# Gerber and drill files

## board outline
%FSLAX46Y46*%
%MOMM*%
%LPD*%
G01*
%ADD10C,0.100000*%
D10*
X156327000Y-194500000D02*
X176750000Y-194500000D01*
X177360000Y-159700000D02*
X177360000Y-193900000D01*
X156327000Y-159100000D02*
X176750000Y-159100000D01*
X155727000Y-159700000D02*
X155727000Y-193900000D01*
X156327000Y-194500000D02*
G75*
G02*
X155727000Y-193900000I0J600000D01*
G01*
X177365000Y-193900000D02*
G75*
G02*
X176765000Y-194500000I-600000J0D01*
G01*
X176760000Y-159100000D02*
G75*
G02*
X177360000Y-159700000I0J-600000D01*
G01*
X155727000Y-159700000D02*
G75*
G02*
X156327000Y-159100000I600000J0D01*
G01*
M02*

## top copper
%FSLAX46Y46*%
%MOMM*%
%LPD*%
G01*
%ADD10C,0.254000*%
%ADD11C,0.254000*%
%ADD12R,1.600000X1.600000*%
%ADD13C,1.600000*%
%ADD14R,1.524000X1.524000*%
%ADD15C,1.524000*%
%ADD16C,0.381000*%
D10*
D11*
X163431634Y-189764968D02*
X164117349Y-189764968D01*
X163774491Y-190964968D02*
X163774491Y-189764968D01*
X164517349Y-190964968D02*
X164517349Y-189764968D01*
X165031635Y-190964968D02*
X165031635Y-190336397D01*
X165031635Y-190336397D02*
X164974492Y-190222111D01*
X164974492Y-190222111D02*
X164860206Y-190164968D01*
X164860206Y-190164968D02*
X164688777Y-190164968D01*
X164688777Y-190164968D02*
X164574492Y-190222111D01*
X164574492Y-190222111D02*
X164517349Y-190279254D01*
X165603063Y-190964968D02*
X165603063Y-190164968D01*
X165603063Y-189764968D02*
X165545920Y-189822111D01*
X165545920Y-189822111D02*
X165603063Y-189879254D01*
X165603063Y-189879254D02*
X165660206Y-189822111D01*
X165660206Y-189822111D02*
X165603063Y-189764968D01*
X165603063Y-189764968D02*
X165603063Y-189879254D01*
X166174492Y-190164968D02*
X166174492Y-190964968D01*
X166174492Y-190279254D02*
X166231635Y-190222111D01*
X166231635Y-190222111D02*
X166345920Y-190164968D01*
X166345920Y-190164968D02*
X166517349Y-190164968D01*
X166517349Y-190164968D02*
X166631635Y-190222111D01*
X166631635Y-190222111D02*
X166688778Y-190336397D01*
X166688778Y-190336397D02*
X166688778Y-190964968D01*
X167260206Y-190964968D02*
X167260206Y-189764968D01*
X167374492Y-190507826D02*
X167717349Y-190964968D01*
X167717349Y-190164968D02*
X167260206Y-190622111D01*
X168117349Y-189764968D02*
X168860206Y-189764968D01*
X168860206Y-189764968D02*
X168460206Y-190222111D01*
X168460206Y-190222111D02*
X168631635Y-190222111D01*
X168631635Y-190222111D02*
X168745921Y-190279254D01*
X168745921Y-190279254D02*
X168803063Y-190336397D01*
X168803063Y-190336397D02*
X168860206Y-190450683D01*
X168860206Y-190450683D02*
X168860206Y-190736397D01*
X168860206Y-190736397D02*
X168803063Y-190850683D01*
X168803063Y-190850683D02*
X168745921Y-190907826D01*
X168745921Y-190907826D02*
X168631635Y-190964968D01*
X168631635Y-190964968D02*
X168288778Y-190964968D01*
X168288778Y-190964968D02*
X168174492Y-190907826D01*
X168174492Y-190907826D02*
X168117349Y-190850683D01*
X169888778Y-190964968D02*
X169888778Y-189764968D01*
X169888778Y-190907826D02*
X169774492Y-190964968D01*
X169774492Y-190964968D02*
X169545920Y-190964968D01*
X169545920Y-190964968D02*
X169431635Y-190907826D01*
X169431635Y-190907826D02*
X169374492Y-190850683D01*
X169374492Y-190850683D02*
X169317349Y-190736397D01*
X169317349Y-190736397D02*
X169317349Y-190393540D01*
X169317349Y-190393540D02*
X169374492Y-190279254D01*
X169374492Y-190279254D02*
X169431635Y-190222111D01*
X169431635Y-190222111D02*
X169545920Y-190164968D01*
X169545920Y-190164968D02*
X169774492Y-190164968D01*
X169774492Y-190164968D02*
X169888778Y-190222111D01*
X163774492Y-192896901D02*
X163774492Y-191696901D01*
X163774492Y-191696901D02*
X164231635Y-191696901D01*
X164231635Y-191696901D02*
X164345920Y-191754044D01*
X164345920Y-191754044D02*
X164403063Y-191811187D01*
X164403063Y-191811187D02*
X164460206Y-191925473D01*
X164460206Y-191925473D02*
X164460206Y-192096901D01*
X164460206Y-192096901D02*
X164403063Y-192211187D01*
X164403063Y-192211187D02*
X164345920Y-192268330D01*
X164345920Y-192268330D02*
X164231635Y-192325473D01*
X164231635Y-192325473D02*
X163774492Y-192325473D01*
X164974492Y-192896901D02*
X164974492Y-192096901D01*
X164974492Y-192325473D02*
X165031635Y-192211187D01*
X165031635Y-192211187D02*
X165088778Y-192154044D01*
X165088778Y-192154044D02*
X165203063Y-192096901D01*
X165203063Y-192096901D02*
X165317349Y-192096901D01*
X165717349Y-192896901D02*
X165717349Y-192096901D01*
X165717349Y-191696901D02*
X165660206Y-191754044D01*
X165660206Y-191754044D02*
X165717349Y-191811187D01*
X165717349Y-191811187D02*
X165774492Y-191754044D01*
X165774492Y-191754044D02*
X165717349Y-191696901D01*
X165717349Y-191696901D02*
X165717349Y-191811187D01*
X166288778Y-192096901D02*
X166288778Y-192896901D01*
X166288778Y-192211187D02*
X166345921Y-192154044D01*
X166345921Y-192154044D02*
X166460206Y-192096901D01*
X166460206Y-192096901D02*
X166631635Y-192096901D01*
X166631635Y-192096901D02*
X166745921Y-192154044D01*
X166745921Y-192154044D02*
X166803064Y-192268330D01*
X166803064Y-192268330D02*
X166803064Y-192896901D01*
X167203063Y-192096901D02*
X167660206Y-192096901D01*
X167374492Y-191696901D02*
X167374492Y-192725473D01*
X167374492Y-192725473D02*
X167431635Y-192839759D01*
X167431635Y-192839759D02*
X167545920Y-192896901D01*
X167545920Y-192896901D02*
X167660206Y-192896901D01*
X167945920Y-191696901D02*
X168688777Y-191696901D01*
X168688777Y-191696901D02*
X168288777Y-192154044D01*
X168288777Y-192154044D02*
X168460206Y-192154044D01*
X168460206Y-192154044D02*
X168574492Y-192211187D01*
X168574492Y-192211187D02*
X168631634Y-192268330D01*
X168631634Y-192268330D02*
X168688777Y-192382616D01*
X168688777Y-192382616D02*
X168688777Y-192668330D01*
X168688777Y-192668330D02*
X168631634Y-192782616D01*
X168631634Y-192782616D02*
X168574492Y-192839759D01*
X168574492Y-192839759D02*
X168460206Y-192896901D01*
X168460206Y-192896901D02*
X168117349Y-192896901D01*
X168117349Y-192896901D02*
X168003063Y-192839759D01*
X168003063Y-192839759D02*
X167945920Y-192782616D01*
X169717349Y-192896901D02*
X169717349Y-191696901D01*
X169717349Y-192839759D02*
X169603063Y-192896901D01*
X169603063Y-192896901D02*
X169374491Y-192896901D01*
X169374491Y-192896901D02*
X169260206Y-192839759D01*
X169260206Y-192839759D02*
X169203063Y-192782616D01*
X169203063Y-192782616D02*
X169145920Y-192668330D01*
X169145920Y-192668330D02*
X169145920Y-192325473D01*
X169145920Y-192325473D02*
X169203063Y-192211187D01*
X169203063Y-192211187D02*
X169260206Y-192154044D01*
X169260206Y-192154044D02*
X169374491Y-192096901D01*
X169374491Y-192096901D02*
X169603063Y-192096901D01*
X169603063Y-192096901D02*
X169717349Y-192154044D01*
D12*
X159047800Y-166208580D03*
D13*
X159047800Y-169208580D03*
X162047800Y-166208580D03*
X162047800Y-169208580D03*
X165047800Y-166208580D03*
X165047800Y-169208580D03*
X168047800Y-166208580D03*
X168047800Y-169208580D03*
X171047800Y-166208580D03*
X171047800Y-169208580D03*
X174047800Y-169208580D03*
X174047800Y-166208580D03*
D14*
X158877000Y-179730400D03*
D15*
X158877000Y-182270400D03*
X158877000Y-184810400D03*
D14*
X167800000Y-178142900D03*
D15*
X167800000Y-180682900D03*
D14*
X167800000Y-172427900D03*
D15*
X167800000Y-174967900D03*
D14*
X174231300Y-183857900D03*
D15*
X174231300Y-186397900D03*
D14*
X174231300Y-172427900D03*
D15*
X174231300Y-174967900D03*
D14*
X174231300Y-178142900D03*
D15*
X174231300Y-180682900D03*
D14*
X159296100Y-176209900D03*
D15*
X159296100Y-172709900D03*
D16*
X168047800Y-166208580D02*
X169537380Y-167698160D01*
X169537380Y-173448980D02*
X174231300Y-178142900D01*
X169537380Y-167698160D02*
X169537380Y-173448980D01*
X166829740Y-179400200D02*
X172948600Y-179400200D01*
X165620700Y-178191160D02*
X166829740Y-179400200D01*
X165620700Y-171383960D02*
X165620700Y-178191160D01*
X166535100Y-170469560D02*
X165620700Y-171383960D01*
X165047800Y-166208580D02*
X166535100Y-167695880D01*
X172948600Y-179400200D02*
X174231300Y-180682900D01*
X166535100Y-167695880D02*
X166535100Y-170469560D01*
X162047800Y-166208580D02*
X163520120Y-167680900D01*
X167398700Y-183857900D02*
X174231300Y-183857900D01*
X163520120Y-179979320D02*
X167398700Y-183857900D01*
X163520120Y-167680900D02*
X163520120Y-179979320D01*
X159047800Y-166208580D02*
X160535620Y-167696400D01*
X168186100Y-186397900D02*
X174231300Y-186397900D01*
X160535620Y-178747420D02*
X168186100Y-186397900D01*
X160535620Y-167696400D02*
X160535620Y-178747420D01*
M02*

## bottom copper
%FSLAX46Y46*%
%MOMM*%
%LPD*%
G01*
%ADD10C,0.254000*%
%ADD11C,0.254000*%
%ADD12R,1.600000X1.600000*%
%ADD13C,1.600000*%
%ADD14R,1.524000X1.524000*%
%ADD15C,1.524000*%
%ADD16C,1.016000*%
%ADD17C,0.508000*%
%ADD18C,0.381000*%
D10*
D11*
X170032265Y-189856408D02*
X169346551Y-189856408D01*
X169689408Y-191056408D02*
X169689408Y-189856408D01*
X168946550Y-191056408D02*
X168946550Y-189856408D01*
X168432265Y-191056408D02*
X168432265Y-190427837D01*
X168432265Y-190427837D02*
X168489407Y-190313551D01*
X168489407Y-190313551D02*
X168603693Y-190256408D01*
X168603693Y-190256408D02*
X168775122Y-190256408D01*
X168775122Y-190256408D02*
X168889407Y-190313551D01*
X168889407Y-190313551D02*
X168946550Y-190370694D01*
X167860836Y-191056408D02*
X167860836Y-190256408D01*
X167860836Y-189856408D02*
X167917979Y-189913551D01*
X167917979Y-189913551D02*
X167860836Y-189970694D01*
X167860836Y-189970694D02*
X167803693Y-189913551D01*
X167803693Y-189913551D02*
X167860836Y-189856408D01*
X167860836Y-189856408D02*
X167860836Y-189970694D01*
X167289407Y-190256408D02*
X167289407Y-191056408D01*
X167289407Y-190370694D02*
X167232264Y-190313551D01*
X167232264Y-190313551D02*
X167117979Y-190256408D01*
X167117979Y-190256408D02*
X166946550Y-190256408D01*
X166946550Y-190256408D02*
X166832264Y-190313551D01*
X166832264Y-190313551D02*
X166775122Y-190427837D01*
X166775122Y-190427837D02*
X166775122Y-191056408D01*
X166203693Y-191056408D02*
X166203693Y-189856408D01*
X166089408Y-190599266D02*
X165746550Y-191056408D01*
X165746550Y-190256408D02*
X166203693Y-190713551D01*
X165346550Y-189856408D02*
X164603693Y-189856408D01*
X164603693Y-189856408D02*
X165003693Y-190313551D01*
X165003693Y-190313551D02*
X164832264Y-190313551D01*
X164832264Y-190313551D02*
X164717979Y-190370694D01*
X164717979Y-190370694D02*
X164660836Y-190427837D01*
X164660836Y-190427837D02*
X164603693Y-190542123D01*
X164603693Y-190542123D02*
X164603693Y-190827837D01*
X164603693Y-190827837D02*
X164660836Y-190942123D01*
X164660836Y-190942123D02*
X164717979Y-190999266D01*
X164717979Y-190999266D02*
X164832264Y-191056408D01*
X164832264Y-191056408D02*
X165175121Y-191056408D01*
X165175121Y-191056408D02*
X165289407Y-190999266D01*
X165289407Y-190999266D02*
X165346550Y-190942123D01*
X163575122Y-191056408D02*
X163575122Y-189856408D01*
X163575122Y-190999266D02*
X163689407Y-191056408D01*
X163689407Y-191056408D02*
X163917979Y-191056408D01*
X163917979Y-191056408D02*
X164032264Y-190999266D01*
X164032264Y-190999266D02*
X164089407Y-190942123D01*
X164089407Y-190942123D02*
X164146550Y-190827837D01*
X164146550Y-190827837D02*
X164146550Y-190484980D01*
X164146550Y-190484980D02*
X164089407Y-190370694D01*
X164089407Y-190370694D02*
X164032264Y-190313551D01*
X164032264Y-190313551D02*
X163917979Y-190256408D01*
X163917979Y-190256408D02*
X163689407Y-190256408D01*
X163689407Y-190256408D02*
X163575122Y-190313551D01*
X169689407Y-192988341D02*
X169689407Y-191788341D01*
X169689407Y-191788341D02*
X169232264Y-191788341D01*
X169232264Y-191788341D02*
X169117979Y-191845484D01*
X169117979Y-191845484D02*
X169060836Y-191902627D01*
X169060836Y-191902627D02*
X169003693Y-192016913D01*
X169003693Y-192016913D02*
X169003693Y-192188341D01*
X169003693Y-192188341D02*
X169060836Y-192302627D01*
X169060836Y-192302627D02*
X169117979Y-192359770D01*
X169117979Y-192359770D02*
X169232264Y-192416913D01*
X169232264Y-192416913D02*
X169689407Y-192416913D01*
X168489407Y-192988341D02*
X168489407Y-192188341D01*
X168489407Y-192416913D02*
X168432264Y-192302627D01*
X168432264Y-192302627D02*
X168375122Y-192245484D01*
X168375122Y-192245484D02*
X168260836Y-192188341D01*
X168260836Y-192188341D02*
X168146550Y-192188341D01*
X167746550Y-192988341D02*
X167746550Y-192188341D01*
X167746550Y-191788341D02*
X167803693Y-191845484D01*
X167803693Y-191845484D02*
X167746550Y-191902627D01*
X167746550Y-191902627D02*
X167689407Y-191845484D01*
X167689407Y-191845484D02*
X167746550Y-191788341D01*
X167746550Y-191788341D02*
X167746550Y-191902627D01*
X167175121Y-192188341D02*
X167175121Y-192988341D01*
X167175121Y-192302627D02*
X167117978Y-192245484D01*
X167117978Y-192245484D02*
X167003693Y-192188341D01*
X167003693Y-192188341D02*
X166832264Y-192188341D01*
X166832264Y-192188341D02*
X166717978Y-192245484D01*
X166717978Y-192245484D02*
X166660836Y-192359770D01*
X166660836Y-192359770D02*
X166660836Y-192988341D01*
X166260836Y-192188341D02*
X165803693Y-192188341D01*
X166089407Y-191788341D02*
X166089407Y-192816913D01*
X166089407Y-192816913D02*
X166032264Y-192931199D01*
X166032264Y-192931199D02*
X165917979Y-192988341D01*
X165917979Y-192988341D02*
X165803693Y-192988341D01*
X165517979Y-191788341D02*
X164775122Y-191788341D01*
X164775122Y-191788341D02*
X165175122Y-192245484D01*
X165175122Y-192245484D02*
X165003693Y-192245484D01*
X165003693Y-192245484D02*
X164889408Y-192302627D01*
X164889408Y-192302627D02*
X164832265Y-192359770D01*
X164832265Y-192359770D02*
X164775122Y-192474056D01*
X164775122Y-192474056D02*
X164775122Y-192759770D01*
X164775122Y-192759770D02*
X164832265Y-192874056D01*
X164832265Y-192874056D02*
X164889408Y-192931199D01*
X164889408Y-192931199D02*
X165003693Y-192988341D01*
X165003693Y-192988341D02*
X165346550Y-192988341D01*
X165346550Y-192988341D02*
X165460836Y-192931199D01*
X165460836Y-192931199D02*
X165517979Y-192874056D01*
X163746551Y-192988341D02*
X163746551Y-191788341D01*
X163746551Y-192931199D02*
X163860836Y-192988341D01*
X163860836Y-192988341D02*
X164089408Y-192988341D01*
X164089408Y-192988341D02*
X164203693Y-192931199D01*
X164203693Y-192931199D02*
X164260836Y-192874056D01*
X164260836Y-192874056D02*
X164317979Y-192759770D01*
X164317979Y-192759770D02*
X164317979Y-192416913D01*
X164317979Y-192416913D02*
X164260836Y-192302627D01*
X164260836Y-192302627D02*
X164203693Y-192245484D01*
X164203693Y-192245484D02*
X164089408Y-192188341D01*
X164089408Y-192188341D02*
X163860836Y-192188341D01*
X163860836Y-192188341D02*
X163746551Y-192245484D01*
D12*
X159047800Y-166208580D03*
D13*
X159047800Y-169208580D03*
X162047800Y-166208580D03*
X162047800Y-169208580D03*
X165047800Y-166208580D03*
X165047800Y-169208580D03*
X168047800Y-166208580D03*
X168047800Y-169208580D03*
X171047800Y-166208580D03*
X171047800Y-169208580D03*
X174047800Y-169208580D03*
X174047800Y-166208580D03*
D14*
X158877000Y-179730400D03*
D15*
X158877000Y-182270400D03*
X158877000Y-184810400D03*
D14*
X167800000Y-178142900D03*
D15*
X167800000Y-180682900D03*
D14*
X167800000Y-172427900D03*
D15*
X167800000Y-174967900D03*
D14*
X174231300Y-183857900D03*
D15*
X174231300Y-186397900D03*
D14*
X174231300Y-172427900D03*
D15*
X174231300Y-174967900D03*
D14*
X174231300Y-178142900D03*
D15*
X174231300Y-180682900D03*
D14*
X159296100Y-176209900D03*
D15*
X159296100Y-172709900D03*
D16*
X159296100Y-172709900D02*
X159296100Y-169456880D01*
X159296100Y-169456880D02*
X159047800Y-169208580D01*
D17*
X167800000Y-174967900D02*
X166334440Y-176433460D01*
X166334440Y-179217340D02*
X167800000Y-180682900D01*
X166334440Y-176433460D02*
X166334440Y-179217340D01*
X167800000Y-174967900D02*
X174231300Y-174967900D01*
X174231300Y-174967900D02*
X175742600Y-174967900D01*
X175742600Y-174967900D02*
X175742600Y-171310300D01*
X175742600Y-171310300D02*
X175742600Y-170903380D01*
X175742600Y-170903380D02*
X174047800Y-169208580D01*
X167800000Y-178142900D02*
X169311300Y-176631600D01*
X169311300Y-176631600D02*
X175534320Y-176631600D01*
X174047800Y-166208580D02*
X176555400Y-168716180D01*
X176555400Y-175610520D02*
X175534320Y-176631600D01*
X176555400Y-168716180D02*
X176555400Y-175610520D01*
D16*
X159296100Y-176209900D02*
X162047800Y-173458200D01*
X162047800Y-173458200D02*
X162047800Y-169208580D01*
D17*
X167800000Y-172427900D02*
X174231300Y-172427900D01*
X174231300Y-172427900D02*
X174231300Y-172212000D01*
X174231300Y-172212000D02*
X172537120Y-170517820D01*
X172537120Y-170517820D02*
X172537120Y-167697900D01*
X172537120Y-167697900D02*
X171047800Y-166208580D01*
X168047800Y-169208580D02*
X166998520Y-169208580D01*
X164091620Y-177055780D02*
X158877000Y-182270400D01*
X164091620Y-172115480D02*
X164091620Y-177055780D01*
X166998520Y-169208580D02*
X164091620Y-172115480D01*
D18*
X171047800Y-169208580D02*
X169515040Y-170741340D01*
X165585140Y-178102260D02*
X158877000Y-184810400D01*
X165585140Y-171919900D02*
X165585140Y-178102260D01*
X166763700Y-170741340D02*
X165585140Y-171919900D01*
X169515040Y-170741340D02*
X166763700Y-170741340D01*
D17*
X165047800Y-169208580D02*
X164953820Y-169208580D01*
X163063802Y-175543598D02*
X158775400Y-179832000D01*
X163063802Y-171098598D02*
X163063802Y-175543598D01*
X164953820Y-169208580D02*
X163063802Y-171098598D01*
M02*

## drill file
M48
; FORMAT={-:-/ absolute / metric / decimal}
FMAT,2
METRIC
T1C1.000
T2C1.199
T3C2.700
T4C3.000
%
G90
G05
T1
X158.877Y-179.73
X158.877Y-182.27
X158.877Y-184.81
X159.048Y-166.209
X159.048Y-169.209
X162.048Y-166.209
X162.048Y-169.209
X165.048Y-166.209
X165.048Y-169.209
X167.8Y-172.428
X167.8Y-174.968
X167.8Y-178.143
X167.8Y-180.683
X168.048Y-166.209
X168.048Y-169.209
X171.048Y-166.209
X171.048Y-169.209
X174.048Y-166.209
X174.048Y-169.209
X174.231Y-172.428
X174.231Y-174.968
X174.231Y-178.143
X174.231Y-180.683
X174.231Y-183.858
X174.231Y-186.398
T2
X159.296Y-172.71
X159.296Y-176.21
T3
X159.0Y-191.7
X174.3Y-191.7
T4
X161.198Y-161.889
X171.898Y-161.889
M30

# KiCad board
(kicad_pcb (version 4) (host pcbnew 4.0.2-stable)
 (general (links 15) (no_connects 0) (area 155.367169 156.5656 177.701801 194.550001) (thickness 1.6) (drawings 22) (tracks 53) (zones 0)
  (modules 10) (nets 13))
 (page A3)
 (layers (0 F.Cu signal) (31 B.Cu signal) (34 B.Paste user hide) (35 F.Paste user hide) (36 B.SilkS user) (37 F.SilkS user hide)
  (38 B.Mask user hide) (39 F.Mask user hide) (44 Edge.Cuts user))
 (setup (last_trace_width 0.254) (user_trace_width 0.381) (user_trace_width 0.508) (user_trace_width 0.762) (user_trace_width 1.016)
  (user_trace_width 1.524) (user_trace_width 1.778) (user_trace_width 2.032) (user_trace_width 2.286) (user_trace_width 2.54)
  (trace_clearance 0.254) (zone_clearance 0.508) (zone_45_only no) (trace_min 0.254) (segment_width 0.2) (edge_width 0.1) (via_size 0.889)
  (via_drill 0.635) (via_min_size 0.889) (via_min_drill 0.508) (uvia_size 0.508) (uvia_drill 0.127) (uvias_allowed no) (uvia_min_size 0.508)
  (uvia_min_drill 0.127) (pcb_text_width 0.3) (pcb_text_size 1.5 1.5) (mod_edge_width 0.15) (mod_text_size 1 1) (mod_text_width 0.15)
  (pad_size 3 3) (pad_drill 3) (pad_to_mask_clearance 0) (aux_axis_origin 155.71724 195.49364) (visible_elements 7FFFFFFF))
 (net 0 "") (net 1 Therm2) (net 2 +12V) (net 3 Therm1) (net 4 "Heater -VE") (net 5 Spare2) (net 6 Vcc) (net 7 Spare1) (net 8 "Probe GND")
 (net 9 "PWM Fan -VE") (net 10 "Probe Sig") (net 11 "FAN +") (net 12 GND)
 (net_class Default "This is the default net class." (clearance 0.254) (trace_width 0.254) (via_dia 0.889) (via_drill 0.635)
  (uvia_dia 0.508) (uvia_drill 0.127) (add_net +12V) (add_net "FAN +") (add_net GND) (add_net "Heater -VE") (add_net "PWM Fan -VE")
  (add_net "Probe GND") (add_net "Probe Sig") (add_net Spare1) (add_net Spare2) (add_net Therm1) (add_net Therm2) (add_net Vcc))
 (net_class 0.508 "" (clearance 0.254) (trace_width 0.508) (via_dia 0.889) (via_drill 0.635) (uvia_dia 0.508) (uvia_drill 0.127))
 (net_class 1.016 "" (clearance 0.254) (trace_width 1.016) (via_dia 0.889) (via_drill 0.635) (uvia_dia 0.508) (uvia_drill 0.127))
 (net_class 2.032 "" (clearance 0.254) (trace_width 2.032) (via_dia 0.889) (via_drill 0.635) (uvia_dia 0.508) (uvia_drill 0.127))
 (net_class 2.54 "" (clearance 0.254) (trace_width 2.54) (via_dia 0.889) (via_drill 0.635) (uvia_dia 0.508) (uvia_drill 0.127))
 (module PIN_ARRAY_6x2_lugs (layer F.Cu) (at 166.5478 167.70858)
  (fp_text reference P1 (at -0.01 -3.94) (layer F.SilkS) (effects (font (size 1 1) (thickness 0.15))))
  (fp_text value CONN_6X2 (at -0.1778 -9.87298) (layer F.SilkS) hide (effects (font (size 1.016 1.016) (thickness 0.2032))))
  (pad 1 thru_hole rect (at -7.5 -1.5) (size 1.6 1.6) (drill 1) (layers *.Cu *.Mask F.SilkS) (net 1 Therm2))
  (pad 2 thru_hole circle (at -7.5 1.5) (size 1.6 1.6) (drill 1) (layers *.Cu *.Mask F.SilkS) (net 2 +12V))
  (pad 3 thru_hole circle (at -4.5 -1.5) (size 1.6 1.6) (drill 1) (layers *.Cu *.Mask F.SilkS) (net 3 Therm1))
  (pad 4 thru_hole circle (at -4.5 1.5) (size 1.6 1.6) (drill 1) (layers *.Cu *.Mask F.SilkS) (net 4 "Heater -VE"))
  (pad 5 thru_hole circle (at -1.5 -1.5) (size 1.6 1.6) (drill 1) (layers *.Cu *.Mask F.SilkS) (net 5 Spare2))
  (pad 6 thru_hole circle (at -1.5 1.5) (size 1.6 1.6) (drill 1) (layers *.Cu *.Mask F.SilkS) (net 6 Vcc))
  (pad 7 thru_hole circle (at 1.5 -1.5) (size 1.6 1.6) (drill 1) (layers *.Cu *.Mask F.SilkS) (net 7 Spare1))
  (pad 8 thru_hole circle (at 1.5 1.5) (size 1.6 1.6) (drill 1) (layers *.Cu *.Mask F.SilkS) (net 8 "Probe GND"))
  (pad 9 thru_hole circle (at 4.5 -1.5) (size 1.6 1.6) (drill 1) (layers *.Cu *.Mask F.SilkS) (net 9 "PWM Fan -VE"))
  (pad 10 thru_hole circle (at 4.5 1.5) (size 1.6 1.6) (drill 1) (layers *.Cu *.Mask F.SilkS) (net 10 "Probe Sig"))
  (pad "" np_thru_hole circle (at -5.35 -5.82) (size 3 3) (drill 3) (layers *.Cu *.Mask F.SilkS))
  (pad "" np_thru_hole circle (at 5.35 -5.82) (size 3 3) (drill 3) (layers *.Cu *.Mask F.SilkS))
  (pad 12 thru_hole circle (at 7.5 1.5) (size 1.6 1.6) (drill 1) (layers *.Cu *.Mask F.SilkS) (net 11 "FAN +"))
  (pad 11 thru_hole circle (at 7.5 -1.5) (size 1.6 1.6) (drill 1) (layers *.Cu *.Mask F.SilkS) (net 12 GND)))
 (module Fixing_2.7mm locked (layer F.Cu) (at 160 191.7)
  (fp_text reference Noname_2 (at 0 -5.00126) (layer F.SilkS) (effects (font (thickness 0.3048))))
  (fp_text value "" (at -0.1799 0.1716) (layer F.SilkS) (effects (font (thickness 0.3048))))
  (pad "" np_thru_hole circle (at -1 0) (size 2.7 2.7) (drill 2.7) (layers *.Cu *.Mask F.SilkS)))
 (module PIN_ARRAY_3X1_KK (layer F.Cu) (at 158.877 182.2704 270)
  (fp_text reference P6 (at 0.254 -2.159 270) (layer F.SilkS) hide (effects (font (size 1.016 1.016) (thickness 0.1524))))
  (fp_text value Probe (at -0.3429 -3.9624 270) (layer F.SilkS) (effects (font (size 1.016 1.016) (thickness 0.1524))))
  (pad 1 thru_hole rect (at -2.54 0 270) (size 1.524 1.524) (drill 1) (layers *.Cu *.Mask F.SilkS) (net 6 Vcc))
  (pad 2 thru_hole circle (at 0 0 270) (size 1.524 1.524) (drill 1) (layers *.Cu *.Mask F.SilkS) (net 8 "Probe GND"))
  (pad 3 thru_hole circle (at 2.54 0 270) (size 1.524 1.524) (drill 1) (layers *.Cu *.Mask F.SilkS) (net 10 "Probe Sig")))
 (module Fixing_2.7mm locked (layer F.Cu) (at 174.3 191.7)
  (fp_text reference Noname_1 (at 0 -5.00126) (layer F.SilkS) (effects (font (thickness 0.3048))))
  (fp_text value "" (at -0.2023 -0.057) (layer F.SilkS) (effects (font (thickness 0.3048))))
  (pad "" np_thru_hole circle (at 0 0) (size 2.7 2.7) (drill 2.7) (layers *.Cu *.Mask F.SilkS)))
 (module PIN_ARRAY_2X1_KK (layer F.Cu) (at 167.8 179.4129 270)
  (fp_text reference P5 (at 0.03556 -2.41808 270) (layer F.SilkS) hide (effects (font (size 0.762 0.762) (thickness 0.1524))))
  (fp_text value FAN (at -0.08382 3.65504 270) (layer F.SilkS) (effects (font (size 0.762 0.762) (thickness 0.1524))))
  (pad 1 thru_hole rect (at -1.27 0 270) (size 1.524 1.524) (drill 1) (layers *.Cu *.Mask F.SilkS) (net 12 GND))
  (pad 2 thru_hole circle (at 1.27 0 270) (size 1.524 1.524) (drill 1) (layers *.Cu *.Mask F.SilkS) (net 11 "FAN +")))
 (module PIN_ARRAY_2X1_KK (layer F.Cu) (at 167.8 173.6979 270)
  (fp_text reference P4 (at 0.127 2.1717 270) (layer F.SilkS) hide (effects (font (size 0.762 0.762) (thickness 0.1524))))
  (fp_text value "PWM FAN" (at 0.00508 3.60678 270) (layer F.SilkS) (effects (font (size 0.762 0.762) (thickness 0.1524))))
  (pad 1 thru_hole rect (at -1.27 0 270) (size 1.524 1.524) (drill 1) (layers *.Cu *.Mask F.SilkS) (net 9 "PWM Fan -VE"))
  (pad 2 thru_hole circle (at 1.27 0 270) (size 1.524 1.524) (drill 1) (layers *.Cu *.Mask F.SilkS) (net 11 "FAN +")))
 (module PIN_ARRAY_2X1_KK (layer F.Cu) (at 174.2313 185.1279 270)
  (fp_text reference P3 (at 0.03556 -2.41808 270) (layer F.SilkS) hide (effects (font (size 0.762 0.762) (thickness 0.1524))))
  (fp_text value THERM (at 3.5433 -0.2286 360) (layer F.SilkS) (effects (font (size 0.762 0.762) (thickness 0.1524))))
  (pad 1 thru_hole rect (at -1.27 0 270) (size 1.524 1.524) (drill 1) (layers *.Cu *.Mask F.SilkS) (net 3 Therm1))
  (pad 2 thru_hole circle (at 1.27 0 270) (size 1.524 1.524) (drill 1) (layers *.Cu *.Mask F.SilkS) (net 1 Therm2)))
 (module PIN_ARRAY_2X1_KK (layer F.Cu) (at 174.2313 173.6979 270)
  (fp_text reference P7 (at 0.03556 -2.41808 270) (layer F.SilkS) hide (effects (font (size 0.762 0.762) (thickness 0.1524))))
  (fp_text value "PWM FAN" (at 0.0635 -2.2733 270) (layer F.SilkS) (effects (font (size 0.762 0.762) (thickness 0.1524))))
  (pad 1 thru_hole rect (at -1.27 0 270) (size 1.524 1.524) (drill 1) (layers *.Cu *.Mask F.SilkS) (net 9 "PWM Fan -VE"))
  (pad 2 thru_hole circle (at 1.27 0 270) (size 1.524 1.524) (drill 1) (layers *.Cu *.Mask F.SilkS) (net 11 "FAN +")))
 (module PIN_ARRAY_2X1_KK (layer F.Cu) (at 174.2313 179.4129 270)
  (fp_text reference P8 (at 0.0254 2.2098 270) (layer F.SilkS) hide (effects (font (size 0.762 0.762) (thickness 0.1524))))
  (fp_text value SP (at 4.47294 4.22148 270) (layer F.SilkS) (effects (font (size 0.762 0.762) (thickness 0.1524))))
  (pad 1 thru_hole rect (at -1.27 0 270) (size 1.524 1.524) (drill 1) (layers *.Cu *.Mask F.SilkS) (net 7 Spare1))
  (pad 2 thru_hole circle (at 1.27 0 270) (size 1.524 1.524) (drill 1) (layers *.Cu *.Mask F.SilkS) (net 5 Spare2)))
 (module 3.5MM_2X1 (layer F.Cu) (at 159.2961 174.4599 90)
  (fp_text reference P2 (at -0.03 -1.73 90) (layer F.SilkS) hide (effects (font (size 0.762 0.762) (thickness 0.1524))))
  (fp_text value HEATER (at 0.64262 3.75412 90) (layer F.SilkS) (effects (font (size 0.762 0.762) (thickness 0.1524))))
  (pad 1 thru_hole rect (at -1.75 0 90) (size 1.524 1.524) (drill 1.19888) (layers *.Cu *.Mask F.SilkS) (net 4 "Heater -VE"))
  (pad 2 thru_hole circle (at 1.75 0 90) (size 1.524 1.524) (drill 1.19888) (layers *.Cu *.Mask F.SilkS) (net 2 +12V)))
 (gr_line (start 156.327 194.5) (end 176.75 194.5) (angle 90) (layer Edge.Cuts) (width 0.1))
 (gr_line (start 177.36 159.7) (end 177.36 193.9) (angle 90) (layer Edge.Cuts) (width 0.1))
 (gr_line (start 156.327 159.1) (end 176.75 159.1) (angle 90) (layer Edge.Cuts) (width 0.1))
 (gr_line (start 155.727 159.7) (end 155.727 193.9) (angle 90) (layer Edge.Cuts) (width 0.1))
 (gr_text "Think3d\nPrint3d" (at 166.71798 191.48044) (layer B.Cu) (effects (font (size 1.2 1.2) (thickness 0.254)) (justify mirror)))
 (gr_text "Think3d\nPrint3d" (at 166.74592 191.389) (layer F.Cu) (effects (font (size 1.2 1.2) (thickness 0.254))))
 (gr_arc (start 156.327 193.9) (end 156.327 194.5) (angle 90) (layer Edge.Cuts) (width 0.1))
 (gr_arc (start 176.765 193.9) (end 177.365 193.9) (angle 90) (layer Edge.Cuts) (width 0.1))
 (gr_arc (start 176.76 159.7) (end 176.76 159.1) (angle 90) (layer Edge.Cuts) (width 0.1))
 (gr_arc (start 156.327 159.7) (end 155.727 159.7) (angle 90) (layer Edge.Cuts) (width 0.1))
 (segment (start 159.2961 172.7099) (end 159.2961 169.45688) (width 1.016) (layer B.Cu) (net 2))
 (segment (start 159.2961 169.45688) (end 159.0478 169.20858) (width 1.016) (layer B.Cu) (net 2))
 (segment (start 167.8 174.9679) (end 166.33444 176.43346) (width 0.508) (layer B.Cu) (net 11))
 (segment (start 166.33444 179.21734) (end 167.8 180.6829) (width 0.508) (layer B.Cu) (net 11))
 (segment (start 166.33444 176.43346) (end 166.33444 179.21734) (width 0.508) (layer B.Cu) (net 11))
 (segment (start 167.8 174.9679) (end 174.2313 174.9679) (width 0.508) (layer B.Cu) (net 11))
 (segment (start 174.2313 174.9679) (end 175.7426 174.9679) (width 0.508) (layer B.Cu) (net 11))
 (segment (start 175.7426 174.9679) (end 175.7426 171.3103) (width 0.508) (layer B.Cu) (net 11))
 (segment (start 175.7426 171.3103) (end 175.7426 170.90338) (width 0.508) (layer B.Cu) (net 11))
 (segment (start 175.7426 170.90338) (end 174.0478 169.20858) (width 0.508) (layer B.Cu) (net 11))
 (segment (start 167.8 178.1429) (end 169.3113 176.6316) (width 0.508) (layer B.Cu) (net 12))
 (segment (start 169.3113 176.6316) (end 175.53432 176.6316) (width 0.508) (layer B.Cu) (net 12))
 (segment (start 174.0478 166.20858) (end 176.5554 168.71618) (width 0.508) (layer B.Cu) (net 12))
 (segment (start 176.5554 175.61052) (end 175.53432 176.6316) (width 0.508) (layer B.Cu) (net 12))
 (segment (start 176.5554 168.71618) (end 176.5554 175.61052) (width 0.508) (layer B.Cu) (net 12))
 (segment (start 159.2961 176.2099) (end 162.0478 173.4582) (width 1.016) (layer B.Cu) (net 4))
 (segment (start 162.0478 173.4582) (end 162.0478 169.20858) (width 1.016) (layer B.Cu) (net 4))
 (segment (start 167.8 172.4279) (end 174.2313 172.4279) (width 0.508) (layer B.Cu) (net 9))
 (segment (start 174.2313 172.4279) (end 174.2313 172.212) (width 0.508) (layer B.Cu) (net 9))
 (segment (start 174.2313 172.212) (end 172.53712 170.51782) (width 0.508) (layer B.Cu) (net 9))
 (segment (start 172.53712 170.51782) (end 172.53712 167.6979) (width 0.508) (layer B.Cu) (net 9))
 (segment (start 172.53712 167.6979) (end 171.0478 166.20858) (width 0.508) (layer B.Cu) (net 9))
 (segment (start 168.0478 169.20858) (end 166.99852 169.20858) (width 0.508) (layer B.Cu) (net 8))
 (segment (start 164.09162 177.05578) (end 158.877 182.2704) (width 0.508) (layer B.Cu) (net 8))
 (segment (start 164.09162 172.11548) (end 164.09162 177.05578) (width 0.508) (layer B.Cu) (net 8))
 (segment (start 166.99852 169.20858) (end 164.09162 172.11548) (width 0.508) (layer B.Cu) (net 8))
 (segment (start 171.0478 169.20858) (end 169.51504 170.74134) (width 0.381) (layer B.Cu) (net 10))
 (segment (start 165.58514 178.10226) (end 158.877 184.8104) (width 0.381) (layer B.Cu) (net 10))
 (segment (start 165.58514 171.9199) (end 165.58514 178.10226) (width 0.381) (layer B.Cu) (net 10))
 (segment (start 166.7637 170.74134) (end 165.58514 171.9199) (width 0.381) (layer B.Cu) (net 10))
 (segment (start 169.51504 170.74134) (end 166.7637 170.74134) (width 0.381) (layer B.Cu) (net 10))
 (segment (start 168.0478 166.20858) (end 169.53738 167.69816) (width 0.381) (layer F.Cu) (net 7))
 (segment (start 169.53738 173.44898) (end 174.2313 178.1429) (width 0.381) (layer F.Cu) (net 7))
 (segment (start 169.53738 167.69816) (end 169.53738 173.44898) (width 0.381) (layer F.Cu) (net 7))
 (segment (start 166.82974 179.4002) (end 172.9486 179.4002) (width 0.381) (layer F.Cu) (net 5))
 (segment (start 165.6207 178.19116) (end 166.82974 179.4002) (width 0.381) (layer F.Cu) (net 5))
 (segment (start 165.6207 171.38396) (end 165.6207 178.19116) (width 0.381) (layer F.Cu) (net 5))
 (segment (start 166.5351 170.46956) (end 165.6207 171.38396) (width 0.381) (layer F.Cu) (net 5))
 (segment (start 165.0478 166.20858) (end 166.5351 167.69588) (width 0.381) (layer F.Cu) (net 5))
 (segment (start 172.9486 179.4002) (end 174.2313 180.6829) (width 0.381) (layer F.Cu) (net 5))
 (segment (start 166.5351 167.69588) (end 166.5351 170.46956) (width 0.381) (layer F.Cu) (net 5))
 (segment (start 162.0478 166.20858) (end 163.52012 167.6809) (width 0.381) (layer F.Cu) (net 3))
 (segment (start 167.3987 183.8579) (end 174.2313 183.8579) (width 0.381) (layer F.Cu) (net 3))
 (segment (start 163.52012 179.97932) (end 167.3987 183.8579) (width 0.381) (layer F.Cu) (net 3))
 (segment (start 163.52012 167.6809) (end 163.52012 179.97932) (width 0.381) (layer F.Cu) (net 3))
 (segment (start 159.0478 166.20858) (end 160.53562 167.6964) (width 0.381) (layer F.Cu) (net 1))
 (segment (start 168.1861 186.3979) (end 174.2313 186.3979) (width 0.381) (layer F.Cu) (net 1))
 (segment (start 160.53562 178.74742) (end 168.1861 186.3979) (width 0.381) (layer F.Cu) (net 1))
 (segment (start 160.53562 167.6964) (end 160.53562 178.74742) (width 0.381) (layer F.Cu) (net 1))
 (segment (start 165.0478 169.20858) (end 164.95382 169.20858) (width 0.508) (layer B.Cu) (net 6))
 (segment (start 163.063802 175.543598) (end 158.7754 179.832) (width 0.508) (layer B.Cu) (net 6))
 (segment (start 163.063802 171.098598) (end 163.063802 175.543598) (width 0.508) (layer B.Cu) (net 6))
 (segment (start 164.95382 169.20858) (end 163.063802 171.098598) (width 0.508) (layer B.Cu) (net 6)))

